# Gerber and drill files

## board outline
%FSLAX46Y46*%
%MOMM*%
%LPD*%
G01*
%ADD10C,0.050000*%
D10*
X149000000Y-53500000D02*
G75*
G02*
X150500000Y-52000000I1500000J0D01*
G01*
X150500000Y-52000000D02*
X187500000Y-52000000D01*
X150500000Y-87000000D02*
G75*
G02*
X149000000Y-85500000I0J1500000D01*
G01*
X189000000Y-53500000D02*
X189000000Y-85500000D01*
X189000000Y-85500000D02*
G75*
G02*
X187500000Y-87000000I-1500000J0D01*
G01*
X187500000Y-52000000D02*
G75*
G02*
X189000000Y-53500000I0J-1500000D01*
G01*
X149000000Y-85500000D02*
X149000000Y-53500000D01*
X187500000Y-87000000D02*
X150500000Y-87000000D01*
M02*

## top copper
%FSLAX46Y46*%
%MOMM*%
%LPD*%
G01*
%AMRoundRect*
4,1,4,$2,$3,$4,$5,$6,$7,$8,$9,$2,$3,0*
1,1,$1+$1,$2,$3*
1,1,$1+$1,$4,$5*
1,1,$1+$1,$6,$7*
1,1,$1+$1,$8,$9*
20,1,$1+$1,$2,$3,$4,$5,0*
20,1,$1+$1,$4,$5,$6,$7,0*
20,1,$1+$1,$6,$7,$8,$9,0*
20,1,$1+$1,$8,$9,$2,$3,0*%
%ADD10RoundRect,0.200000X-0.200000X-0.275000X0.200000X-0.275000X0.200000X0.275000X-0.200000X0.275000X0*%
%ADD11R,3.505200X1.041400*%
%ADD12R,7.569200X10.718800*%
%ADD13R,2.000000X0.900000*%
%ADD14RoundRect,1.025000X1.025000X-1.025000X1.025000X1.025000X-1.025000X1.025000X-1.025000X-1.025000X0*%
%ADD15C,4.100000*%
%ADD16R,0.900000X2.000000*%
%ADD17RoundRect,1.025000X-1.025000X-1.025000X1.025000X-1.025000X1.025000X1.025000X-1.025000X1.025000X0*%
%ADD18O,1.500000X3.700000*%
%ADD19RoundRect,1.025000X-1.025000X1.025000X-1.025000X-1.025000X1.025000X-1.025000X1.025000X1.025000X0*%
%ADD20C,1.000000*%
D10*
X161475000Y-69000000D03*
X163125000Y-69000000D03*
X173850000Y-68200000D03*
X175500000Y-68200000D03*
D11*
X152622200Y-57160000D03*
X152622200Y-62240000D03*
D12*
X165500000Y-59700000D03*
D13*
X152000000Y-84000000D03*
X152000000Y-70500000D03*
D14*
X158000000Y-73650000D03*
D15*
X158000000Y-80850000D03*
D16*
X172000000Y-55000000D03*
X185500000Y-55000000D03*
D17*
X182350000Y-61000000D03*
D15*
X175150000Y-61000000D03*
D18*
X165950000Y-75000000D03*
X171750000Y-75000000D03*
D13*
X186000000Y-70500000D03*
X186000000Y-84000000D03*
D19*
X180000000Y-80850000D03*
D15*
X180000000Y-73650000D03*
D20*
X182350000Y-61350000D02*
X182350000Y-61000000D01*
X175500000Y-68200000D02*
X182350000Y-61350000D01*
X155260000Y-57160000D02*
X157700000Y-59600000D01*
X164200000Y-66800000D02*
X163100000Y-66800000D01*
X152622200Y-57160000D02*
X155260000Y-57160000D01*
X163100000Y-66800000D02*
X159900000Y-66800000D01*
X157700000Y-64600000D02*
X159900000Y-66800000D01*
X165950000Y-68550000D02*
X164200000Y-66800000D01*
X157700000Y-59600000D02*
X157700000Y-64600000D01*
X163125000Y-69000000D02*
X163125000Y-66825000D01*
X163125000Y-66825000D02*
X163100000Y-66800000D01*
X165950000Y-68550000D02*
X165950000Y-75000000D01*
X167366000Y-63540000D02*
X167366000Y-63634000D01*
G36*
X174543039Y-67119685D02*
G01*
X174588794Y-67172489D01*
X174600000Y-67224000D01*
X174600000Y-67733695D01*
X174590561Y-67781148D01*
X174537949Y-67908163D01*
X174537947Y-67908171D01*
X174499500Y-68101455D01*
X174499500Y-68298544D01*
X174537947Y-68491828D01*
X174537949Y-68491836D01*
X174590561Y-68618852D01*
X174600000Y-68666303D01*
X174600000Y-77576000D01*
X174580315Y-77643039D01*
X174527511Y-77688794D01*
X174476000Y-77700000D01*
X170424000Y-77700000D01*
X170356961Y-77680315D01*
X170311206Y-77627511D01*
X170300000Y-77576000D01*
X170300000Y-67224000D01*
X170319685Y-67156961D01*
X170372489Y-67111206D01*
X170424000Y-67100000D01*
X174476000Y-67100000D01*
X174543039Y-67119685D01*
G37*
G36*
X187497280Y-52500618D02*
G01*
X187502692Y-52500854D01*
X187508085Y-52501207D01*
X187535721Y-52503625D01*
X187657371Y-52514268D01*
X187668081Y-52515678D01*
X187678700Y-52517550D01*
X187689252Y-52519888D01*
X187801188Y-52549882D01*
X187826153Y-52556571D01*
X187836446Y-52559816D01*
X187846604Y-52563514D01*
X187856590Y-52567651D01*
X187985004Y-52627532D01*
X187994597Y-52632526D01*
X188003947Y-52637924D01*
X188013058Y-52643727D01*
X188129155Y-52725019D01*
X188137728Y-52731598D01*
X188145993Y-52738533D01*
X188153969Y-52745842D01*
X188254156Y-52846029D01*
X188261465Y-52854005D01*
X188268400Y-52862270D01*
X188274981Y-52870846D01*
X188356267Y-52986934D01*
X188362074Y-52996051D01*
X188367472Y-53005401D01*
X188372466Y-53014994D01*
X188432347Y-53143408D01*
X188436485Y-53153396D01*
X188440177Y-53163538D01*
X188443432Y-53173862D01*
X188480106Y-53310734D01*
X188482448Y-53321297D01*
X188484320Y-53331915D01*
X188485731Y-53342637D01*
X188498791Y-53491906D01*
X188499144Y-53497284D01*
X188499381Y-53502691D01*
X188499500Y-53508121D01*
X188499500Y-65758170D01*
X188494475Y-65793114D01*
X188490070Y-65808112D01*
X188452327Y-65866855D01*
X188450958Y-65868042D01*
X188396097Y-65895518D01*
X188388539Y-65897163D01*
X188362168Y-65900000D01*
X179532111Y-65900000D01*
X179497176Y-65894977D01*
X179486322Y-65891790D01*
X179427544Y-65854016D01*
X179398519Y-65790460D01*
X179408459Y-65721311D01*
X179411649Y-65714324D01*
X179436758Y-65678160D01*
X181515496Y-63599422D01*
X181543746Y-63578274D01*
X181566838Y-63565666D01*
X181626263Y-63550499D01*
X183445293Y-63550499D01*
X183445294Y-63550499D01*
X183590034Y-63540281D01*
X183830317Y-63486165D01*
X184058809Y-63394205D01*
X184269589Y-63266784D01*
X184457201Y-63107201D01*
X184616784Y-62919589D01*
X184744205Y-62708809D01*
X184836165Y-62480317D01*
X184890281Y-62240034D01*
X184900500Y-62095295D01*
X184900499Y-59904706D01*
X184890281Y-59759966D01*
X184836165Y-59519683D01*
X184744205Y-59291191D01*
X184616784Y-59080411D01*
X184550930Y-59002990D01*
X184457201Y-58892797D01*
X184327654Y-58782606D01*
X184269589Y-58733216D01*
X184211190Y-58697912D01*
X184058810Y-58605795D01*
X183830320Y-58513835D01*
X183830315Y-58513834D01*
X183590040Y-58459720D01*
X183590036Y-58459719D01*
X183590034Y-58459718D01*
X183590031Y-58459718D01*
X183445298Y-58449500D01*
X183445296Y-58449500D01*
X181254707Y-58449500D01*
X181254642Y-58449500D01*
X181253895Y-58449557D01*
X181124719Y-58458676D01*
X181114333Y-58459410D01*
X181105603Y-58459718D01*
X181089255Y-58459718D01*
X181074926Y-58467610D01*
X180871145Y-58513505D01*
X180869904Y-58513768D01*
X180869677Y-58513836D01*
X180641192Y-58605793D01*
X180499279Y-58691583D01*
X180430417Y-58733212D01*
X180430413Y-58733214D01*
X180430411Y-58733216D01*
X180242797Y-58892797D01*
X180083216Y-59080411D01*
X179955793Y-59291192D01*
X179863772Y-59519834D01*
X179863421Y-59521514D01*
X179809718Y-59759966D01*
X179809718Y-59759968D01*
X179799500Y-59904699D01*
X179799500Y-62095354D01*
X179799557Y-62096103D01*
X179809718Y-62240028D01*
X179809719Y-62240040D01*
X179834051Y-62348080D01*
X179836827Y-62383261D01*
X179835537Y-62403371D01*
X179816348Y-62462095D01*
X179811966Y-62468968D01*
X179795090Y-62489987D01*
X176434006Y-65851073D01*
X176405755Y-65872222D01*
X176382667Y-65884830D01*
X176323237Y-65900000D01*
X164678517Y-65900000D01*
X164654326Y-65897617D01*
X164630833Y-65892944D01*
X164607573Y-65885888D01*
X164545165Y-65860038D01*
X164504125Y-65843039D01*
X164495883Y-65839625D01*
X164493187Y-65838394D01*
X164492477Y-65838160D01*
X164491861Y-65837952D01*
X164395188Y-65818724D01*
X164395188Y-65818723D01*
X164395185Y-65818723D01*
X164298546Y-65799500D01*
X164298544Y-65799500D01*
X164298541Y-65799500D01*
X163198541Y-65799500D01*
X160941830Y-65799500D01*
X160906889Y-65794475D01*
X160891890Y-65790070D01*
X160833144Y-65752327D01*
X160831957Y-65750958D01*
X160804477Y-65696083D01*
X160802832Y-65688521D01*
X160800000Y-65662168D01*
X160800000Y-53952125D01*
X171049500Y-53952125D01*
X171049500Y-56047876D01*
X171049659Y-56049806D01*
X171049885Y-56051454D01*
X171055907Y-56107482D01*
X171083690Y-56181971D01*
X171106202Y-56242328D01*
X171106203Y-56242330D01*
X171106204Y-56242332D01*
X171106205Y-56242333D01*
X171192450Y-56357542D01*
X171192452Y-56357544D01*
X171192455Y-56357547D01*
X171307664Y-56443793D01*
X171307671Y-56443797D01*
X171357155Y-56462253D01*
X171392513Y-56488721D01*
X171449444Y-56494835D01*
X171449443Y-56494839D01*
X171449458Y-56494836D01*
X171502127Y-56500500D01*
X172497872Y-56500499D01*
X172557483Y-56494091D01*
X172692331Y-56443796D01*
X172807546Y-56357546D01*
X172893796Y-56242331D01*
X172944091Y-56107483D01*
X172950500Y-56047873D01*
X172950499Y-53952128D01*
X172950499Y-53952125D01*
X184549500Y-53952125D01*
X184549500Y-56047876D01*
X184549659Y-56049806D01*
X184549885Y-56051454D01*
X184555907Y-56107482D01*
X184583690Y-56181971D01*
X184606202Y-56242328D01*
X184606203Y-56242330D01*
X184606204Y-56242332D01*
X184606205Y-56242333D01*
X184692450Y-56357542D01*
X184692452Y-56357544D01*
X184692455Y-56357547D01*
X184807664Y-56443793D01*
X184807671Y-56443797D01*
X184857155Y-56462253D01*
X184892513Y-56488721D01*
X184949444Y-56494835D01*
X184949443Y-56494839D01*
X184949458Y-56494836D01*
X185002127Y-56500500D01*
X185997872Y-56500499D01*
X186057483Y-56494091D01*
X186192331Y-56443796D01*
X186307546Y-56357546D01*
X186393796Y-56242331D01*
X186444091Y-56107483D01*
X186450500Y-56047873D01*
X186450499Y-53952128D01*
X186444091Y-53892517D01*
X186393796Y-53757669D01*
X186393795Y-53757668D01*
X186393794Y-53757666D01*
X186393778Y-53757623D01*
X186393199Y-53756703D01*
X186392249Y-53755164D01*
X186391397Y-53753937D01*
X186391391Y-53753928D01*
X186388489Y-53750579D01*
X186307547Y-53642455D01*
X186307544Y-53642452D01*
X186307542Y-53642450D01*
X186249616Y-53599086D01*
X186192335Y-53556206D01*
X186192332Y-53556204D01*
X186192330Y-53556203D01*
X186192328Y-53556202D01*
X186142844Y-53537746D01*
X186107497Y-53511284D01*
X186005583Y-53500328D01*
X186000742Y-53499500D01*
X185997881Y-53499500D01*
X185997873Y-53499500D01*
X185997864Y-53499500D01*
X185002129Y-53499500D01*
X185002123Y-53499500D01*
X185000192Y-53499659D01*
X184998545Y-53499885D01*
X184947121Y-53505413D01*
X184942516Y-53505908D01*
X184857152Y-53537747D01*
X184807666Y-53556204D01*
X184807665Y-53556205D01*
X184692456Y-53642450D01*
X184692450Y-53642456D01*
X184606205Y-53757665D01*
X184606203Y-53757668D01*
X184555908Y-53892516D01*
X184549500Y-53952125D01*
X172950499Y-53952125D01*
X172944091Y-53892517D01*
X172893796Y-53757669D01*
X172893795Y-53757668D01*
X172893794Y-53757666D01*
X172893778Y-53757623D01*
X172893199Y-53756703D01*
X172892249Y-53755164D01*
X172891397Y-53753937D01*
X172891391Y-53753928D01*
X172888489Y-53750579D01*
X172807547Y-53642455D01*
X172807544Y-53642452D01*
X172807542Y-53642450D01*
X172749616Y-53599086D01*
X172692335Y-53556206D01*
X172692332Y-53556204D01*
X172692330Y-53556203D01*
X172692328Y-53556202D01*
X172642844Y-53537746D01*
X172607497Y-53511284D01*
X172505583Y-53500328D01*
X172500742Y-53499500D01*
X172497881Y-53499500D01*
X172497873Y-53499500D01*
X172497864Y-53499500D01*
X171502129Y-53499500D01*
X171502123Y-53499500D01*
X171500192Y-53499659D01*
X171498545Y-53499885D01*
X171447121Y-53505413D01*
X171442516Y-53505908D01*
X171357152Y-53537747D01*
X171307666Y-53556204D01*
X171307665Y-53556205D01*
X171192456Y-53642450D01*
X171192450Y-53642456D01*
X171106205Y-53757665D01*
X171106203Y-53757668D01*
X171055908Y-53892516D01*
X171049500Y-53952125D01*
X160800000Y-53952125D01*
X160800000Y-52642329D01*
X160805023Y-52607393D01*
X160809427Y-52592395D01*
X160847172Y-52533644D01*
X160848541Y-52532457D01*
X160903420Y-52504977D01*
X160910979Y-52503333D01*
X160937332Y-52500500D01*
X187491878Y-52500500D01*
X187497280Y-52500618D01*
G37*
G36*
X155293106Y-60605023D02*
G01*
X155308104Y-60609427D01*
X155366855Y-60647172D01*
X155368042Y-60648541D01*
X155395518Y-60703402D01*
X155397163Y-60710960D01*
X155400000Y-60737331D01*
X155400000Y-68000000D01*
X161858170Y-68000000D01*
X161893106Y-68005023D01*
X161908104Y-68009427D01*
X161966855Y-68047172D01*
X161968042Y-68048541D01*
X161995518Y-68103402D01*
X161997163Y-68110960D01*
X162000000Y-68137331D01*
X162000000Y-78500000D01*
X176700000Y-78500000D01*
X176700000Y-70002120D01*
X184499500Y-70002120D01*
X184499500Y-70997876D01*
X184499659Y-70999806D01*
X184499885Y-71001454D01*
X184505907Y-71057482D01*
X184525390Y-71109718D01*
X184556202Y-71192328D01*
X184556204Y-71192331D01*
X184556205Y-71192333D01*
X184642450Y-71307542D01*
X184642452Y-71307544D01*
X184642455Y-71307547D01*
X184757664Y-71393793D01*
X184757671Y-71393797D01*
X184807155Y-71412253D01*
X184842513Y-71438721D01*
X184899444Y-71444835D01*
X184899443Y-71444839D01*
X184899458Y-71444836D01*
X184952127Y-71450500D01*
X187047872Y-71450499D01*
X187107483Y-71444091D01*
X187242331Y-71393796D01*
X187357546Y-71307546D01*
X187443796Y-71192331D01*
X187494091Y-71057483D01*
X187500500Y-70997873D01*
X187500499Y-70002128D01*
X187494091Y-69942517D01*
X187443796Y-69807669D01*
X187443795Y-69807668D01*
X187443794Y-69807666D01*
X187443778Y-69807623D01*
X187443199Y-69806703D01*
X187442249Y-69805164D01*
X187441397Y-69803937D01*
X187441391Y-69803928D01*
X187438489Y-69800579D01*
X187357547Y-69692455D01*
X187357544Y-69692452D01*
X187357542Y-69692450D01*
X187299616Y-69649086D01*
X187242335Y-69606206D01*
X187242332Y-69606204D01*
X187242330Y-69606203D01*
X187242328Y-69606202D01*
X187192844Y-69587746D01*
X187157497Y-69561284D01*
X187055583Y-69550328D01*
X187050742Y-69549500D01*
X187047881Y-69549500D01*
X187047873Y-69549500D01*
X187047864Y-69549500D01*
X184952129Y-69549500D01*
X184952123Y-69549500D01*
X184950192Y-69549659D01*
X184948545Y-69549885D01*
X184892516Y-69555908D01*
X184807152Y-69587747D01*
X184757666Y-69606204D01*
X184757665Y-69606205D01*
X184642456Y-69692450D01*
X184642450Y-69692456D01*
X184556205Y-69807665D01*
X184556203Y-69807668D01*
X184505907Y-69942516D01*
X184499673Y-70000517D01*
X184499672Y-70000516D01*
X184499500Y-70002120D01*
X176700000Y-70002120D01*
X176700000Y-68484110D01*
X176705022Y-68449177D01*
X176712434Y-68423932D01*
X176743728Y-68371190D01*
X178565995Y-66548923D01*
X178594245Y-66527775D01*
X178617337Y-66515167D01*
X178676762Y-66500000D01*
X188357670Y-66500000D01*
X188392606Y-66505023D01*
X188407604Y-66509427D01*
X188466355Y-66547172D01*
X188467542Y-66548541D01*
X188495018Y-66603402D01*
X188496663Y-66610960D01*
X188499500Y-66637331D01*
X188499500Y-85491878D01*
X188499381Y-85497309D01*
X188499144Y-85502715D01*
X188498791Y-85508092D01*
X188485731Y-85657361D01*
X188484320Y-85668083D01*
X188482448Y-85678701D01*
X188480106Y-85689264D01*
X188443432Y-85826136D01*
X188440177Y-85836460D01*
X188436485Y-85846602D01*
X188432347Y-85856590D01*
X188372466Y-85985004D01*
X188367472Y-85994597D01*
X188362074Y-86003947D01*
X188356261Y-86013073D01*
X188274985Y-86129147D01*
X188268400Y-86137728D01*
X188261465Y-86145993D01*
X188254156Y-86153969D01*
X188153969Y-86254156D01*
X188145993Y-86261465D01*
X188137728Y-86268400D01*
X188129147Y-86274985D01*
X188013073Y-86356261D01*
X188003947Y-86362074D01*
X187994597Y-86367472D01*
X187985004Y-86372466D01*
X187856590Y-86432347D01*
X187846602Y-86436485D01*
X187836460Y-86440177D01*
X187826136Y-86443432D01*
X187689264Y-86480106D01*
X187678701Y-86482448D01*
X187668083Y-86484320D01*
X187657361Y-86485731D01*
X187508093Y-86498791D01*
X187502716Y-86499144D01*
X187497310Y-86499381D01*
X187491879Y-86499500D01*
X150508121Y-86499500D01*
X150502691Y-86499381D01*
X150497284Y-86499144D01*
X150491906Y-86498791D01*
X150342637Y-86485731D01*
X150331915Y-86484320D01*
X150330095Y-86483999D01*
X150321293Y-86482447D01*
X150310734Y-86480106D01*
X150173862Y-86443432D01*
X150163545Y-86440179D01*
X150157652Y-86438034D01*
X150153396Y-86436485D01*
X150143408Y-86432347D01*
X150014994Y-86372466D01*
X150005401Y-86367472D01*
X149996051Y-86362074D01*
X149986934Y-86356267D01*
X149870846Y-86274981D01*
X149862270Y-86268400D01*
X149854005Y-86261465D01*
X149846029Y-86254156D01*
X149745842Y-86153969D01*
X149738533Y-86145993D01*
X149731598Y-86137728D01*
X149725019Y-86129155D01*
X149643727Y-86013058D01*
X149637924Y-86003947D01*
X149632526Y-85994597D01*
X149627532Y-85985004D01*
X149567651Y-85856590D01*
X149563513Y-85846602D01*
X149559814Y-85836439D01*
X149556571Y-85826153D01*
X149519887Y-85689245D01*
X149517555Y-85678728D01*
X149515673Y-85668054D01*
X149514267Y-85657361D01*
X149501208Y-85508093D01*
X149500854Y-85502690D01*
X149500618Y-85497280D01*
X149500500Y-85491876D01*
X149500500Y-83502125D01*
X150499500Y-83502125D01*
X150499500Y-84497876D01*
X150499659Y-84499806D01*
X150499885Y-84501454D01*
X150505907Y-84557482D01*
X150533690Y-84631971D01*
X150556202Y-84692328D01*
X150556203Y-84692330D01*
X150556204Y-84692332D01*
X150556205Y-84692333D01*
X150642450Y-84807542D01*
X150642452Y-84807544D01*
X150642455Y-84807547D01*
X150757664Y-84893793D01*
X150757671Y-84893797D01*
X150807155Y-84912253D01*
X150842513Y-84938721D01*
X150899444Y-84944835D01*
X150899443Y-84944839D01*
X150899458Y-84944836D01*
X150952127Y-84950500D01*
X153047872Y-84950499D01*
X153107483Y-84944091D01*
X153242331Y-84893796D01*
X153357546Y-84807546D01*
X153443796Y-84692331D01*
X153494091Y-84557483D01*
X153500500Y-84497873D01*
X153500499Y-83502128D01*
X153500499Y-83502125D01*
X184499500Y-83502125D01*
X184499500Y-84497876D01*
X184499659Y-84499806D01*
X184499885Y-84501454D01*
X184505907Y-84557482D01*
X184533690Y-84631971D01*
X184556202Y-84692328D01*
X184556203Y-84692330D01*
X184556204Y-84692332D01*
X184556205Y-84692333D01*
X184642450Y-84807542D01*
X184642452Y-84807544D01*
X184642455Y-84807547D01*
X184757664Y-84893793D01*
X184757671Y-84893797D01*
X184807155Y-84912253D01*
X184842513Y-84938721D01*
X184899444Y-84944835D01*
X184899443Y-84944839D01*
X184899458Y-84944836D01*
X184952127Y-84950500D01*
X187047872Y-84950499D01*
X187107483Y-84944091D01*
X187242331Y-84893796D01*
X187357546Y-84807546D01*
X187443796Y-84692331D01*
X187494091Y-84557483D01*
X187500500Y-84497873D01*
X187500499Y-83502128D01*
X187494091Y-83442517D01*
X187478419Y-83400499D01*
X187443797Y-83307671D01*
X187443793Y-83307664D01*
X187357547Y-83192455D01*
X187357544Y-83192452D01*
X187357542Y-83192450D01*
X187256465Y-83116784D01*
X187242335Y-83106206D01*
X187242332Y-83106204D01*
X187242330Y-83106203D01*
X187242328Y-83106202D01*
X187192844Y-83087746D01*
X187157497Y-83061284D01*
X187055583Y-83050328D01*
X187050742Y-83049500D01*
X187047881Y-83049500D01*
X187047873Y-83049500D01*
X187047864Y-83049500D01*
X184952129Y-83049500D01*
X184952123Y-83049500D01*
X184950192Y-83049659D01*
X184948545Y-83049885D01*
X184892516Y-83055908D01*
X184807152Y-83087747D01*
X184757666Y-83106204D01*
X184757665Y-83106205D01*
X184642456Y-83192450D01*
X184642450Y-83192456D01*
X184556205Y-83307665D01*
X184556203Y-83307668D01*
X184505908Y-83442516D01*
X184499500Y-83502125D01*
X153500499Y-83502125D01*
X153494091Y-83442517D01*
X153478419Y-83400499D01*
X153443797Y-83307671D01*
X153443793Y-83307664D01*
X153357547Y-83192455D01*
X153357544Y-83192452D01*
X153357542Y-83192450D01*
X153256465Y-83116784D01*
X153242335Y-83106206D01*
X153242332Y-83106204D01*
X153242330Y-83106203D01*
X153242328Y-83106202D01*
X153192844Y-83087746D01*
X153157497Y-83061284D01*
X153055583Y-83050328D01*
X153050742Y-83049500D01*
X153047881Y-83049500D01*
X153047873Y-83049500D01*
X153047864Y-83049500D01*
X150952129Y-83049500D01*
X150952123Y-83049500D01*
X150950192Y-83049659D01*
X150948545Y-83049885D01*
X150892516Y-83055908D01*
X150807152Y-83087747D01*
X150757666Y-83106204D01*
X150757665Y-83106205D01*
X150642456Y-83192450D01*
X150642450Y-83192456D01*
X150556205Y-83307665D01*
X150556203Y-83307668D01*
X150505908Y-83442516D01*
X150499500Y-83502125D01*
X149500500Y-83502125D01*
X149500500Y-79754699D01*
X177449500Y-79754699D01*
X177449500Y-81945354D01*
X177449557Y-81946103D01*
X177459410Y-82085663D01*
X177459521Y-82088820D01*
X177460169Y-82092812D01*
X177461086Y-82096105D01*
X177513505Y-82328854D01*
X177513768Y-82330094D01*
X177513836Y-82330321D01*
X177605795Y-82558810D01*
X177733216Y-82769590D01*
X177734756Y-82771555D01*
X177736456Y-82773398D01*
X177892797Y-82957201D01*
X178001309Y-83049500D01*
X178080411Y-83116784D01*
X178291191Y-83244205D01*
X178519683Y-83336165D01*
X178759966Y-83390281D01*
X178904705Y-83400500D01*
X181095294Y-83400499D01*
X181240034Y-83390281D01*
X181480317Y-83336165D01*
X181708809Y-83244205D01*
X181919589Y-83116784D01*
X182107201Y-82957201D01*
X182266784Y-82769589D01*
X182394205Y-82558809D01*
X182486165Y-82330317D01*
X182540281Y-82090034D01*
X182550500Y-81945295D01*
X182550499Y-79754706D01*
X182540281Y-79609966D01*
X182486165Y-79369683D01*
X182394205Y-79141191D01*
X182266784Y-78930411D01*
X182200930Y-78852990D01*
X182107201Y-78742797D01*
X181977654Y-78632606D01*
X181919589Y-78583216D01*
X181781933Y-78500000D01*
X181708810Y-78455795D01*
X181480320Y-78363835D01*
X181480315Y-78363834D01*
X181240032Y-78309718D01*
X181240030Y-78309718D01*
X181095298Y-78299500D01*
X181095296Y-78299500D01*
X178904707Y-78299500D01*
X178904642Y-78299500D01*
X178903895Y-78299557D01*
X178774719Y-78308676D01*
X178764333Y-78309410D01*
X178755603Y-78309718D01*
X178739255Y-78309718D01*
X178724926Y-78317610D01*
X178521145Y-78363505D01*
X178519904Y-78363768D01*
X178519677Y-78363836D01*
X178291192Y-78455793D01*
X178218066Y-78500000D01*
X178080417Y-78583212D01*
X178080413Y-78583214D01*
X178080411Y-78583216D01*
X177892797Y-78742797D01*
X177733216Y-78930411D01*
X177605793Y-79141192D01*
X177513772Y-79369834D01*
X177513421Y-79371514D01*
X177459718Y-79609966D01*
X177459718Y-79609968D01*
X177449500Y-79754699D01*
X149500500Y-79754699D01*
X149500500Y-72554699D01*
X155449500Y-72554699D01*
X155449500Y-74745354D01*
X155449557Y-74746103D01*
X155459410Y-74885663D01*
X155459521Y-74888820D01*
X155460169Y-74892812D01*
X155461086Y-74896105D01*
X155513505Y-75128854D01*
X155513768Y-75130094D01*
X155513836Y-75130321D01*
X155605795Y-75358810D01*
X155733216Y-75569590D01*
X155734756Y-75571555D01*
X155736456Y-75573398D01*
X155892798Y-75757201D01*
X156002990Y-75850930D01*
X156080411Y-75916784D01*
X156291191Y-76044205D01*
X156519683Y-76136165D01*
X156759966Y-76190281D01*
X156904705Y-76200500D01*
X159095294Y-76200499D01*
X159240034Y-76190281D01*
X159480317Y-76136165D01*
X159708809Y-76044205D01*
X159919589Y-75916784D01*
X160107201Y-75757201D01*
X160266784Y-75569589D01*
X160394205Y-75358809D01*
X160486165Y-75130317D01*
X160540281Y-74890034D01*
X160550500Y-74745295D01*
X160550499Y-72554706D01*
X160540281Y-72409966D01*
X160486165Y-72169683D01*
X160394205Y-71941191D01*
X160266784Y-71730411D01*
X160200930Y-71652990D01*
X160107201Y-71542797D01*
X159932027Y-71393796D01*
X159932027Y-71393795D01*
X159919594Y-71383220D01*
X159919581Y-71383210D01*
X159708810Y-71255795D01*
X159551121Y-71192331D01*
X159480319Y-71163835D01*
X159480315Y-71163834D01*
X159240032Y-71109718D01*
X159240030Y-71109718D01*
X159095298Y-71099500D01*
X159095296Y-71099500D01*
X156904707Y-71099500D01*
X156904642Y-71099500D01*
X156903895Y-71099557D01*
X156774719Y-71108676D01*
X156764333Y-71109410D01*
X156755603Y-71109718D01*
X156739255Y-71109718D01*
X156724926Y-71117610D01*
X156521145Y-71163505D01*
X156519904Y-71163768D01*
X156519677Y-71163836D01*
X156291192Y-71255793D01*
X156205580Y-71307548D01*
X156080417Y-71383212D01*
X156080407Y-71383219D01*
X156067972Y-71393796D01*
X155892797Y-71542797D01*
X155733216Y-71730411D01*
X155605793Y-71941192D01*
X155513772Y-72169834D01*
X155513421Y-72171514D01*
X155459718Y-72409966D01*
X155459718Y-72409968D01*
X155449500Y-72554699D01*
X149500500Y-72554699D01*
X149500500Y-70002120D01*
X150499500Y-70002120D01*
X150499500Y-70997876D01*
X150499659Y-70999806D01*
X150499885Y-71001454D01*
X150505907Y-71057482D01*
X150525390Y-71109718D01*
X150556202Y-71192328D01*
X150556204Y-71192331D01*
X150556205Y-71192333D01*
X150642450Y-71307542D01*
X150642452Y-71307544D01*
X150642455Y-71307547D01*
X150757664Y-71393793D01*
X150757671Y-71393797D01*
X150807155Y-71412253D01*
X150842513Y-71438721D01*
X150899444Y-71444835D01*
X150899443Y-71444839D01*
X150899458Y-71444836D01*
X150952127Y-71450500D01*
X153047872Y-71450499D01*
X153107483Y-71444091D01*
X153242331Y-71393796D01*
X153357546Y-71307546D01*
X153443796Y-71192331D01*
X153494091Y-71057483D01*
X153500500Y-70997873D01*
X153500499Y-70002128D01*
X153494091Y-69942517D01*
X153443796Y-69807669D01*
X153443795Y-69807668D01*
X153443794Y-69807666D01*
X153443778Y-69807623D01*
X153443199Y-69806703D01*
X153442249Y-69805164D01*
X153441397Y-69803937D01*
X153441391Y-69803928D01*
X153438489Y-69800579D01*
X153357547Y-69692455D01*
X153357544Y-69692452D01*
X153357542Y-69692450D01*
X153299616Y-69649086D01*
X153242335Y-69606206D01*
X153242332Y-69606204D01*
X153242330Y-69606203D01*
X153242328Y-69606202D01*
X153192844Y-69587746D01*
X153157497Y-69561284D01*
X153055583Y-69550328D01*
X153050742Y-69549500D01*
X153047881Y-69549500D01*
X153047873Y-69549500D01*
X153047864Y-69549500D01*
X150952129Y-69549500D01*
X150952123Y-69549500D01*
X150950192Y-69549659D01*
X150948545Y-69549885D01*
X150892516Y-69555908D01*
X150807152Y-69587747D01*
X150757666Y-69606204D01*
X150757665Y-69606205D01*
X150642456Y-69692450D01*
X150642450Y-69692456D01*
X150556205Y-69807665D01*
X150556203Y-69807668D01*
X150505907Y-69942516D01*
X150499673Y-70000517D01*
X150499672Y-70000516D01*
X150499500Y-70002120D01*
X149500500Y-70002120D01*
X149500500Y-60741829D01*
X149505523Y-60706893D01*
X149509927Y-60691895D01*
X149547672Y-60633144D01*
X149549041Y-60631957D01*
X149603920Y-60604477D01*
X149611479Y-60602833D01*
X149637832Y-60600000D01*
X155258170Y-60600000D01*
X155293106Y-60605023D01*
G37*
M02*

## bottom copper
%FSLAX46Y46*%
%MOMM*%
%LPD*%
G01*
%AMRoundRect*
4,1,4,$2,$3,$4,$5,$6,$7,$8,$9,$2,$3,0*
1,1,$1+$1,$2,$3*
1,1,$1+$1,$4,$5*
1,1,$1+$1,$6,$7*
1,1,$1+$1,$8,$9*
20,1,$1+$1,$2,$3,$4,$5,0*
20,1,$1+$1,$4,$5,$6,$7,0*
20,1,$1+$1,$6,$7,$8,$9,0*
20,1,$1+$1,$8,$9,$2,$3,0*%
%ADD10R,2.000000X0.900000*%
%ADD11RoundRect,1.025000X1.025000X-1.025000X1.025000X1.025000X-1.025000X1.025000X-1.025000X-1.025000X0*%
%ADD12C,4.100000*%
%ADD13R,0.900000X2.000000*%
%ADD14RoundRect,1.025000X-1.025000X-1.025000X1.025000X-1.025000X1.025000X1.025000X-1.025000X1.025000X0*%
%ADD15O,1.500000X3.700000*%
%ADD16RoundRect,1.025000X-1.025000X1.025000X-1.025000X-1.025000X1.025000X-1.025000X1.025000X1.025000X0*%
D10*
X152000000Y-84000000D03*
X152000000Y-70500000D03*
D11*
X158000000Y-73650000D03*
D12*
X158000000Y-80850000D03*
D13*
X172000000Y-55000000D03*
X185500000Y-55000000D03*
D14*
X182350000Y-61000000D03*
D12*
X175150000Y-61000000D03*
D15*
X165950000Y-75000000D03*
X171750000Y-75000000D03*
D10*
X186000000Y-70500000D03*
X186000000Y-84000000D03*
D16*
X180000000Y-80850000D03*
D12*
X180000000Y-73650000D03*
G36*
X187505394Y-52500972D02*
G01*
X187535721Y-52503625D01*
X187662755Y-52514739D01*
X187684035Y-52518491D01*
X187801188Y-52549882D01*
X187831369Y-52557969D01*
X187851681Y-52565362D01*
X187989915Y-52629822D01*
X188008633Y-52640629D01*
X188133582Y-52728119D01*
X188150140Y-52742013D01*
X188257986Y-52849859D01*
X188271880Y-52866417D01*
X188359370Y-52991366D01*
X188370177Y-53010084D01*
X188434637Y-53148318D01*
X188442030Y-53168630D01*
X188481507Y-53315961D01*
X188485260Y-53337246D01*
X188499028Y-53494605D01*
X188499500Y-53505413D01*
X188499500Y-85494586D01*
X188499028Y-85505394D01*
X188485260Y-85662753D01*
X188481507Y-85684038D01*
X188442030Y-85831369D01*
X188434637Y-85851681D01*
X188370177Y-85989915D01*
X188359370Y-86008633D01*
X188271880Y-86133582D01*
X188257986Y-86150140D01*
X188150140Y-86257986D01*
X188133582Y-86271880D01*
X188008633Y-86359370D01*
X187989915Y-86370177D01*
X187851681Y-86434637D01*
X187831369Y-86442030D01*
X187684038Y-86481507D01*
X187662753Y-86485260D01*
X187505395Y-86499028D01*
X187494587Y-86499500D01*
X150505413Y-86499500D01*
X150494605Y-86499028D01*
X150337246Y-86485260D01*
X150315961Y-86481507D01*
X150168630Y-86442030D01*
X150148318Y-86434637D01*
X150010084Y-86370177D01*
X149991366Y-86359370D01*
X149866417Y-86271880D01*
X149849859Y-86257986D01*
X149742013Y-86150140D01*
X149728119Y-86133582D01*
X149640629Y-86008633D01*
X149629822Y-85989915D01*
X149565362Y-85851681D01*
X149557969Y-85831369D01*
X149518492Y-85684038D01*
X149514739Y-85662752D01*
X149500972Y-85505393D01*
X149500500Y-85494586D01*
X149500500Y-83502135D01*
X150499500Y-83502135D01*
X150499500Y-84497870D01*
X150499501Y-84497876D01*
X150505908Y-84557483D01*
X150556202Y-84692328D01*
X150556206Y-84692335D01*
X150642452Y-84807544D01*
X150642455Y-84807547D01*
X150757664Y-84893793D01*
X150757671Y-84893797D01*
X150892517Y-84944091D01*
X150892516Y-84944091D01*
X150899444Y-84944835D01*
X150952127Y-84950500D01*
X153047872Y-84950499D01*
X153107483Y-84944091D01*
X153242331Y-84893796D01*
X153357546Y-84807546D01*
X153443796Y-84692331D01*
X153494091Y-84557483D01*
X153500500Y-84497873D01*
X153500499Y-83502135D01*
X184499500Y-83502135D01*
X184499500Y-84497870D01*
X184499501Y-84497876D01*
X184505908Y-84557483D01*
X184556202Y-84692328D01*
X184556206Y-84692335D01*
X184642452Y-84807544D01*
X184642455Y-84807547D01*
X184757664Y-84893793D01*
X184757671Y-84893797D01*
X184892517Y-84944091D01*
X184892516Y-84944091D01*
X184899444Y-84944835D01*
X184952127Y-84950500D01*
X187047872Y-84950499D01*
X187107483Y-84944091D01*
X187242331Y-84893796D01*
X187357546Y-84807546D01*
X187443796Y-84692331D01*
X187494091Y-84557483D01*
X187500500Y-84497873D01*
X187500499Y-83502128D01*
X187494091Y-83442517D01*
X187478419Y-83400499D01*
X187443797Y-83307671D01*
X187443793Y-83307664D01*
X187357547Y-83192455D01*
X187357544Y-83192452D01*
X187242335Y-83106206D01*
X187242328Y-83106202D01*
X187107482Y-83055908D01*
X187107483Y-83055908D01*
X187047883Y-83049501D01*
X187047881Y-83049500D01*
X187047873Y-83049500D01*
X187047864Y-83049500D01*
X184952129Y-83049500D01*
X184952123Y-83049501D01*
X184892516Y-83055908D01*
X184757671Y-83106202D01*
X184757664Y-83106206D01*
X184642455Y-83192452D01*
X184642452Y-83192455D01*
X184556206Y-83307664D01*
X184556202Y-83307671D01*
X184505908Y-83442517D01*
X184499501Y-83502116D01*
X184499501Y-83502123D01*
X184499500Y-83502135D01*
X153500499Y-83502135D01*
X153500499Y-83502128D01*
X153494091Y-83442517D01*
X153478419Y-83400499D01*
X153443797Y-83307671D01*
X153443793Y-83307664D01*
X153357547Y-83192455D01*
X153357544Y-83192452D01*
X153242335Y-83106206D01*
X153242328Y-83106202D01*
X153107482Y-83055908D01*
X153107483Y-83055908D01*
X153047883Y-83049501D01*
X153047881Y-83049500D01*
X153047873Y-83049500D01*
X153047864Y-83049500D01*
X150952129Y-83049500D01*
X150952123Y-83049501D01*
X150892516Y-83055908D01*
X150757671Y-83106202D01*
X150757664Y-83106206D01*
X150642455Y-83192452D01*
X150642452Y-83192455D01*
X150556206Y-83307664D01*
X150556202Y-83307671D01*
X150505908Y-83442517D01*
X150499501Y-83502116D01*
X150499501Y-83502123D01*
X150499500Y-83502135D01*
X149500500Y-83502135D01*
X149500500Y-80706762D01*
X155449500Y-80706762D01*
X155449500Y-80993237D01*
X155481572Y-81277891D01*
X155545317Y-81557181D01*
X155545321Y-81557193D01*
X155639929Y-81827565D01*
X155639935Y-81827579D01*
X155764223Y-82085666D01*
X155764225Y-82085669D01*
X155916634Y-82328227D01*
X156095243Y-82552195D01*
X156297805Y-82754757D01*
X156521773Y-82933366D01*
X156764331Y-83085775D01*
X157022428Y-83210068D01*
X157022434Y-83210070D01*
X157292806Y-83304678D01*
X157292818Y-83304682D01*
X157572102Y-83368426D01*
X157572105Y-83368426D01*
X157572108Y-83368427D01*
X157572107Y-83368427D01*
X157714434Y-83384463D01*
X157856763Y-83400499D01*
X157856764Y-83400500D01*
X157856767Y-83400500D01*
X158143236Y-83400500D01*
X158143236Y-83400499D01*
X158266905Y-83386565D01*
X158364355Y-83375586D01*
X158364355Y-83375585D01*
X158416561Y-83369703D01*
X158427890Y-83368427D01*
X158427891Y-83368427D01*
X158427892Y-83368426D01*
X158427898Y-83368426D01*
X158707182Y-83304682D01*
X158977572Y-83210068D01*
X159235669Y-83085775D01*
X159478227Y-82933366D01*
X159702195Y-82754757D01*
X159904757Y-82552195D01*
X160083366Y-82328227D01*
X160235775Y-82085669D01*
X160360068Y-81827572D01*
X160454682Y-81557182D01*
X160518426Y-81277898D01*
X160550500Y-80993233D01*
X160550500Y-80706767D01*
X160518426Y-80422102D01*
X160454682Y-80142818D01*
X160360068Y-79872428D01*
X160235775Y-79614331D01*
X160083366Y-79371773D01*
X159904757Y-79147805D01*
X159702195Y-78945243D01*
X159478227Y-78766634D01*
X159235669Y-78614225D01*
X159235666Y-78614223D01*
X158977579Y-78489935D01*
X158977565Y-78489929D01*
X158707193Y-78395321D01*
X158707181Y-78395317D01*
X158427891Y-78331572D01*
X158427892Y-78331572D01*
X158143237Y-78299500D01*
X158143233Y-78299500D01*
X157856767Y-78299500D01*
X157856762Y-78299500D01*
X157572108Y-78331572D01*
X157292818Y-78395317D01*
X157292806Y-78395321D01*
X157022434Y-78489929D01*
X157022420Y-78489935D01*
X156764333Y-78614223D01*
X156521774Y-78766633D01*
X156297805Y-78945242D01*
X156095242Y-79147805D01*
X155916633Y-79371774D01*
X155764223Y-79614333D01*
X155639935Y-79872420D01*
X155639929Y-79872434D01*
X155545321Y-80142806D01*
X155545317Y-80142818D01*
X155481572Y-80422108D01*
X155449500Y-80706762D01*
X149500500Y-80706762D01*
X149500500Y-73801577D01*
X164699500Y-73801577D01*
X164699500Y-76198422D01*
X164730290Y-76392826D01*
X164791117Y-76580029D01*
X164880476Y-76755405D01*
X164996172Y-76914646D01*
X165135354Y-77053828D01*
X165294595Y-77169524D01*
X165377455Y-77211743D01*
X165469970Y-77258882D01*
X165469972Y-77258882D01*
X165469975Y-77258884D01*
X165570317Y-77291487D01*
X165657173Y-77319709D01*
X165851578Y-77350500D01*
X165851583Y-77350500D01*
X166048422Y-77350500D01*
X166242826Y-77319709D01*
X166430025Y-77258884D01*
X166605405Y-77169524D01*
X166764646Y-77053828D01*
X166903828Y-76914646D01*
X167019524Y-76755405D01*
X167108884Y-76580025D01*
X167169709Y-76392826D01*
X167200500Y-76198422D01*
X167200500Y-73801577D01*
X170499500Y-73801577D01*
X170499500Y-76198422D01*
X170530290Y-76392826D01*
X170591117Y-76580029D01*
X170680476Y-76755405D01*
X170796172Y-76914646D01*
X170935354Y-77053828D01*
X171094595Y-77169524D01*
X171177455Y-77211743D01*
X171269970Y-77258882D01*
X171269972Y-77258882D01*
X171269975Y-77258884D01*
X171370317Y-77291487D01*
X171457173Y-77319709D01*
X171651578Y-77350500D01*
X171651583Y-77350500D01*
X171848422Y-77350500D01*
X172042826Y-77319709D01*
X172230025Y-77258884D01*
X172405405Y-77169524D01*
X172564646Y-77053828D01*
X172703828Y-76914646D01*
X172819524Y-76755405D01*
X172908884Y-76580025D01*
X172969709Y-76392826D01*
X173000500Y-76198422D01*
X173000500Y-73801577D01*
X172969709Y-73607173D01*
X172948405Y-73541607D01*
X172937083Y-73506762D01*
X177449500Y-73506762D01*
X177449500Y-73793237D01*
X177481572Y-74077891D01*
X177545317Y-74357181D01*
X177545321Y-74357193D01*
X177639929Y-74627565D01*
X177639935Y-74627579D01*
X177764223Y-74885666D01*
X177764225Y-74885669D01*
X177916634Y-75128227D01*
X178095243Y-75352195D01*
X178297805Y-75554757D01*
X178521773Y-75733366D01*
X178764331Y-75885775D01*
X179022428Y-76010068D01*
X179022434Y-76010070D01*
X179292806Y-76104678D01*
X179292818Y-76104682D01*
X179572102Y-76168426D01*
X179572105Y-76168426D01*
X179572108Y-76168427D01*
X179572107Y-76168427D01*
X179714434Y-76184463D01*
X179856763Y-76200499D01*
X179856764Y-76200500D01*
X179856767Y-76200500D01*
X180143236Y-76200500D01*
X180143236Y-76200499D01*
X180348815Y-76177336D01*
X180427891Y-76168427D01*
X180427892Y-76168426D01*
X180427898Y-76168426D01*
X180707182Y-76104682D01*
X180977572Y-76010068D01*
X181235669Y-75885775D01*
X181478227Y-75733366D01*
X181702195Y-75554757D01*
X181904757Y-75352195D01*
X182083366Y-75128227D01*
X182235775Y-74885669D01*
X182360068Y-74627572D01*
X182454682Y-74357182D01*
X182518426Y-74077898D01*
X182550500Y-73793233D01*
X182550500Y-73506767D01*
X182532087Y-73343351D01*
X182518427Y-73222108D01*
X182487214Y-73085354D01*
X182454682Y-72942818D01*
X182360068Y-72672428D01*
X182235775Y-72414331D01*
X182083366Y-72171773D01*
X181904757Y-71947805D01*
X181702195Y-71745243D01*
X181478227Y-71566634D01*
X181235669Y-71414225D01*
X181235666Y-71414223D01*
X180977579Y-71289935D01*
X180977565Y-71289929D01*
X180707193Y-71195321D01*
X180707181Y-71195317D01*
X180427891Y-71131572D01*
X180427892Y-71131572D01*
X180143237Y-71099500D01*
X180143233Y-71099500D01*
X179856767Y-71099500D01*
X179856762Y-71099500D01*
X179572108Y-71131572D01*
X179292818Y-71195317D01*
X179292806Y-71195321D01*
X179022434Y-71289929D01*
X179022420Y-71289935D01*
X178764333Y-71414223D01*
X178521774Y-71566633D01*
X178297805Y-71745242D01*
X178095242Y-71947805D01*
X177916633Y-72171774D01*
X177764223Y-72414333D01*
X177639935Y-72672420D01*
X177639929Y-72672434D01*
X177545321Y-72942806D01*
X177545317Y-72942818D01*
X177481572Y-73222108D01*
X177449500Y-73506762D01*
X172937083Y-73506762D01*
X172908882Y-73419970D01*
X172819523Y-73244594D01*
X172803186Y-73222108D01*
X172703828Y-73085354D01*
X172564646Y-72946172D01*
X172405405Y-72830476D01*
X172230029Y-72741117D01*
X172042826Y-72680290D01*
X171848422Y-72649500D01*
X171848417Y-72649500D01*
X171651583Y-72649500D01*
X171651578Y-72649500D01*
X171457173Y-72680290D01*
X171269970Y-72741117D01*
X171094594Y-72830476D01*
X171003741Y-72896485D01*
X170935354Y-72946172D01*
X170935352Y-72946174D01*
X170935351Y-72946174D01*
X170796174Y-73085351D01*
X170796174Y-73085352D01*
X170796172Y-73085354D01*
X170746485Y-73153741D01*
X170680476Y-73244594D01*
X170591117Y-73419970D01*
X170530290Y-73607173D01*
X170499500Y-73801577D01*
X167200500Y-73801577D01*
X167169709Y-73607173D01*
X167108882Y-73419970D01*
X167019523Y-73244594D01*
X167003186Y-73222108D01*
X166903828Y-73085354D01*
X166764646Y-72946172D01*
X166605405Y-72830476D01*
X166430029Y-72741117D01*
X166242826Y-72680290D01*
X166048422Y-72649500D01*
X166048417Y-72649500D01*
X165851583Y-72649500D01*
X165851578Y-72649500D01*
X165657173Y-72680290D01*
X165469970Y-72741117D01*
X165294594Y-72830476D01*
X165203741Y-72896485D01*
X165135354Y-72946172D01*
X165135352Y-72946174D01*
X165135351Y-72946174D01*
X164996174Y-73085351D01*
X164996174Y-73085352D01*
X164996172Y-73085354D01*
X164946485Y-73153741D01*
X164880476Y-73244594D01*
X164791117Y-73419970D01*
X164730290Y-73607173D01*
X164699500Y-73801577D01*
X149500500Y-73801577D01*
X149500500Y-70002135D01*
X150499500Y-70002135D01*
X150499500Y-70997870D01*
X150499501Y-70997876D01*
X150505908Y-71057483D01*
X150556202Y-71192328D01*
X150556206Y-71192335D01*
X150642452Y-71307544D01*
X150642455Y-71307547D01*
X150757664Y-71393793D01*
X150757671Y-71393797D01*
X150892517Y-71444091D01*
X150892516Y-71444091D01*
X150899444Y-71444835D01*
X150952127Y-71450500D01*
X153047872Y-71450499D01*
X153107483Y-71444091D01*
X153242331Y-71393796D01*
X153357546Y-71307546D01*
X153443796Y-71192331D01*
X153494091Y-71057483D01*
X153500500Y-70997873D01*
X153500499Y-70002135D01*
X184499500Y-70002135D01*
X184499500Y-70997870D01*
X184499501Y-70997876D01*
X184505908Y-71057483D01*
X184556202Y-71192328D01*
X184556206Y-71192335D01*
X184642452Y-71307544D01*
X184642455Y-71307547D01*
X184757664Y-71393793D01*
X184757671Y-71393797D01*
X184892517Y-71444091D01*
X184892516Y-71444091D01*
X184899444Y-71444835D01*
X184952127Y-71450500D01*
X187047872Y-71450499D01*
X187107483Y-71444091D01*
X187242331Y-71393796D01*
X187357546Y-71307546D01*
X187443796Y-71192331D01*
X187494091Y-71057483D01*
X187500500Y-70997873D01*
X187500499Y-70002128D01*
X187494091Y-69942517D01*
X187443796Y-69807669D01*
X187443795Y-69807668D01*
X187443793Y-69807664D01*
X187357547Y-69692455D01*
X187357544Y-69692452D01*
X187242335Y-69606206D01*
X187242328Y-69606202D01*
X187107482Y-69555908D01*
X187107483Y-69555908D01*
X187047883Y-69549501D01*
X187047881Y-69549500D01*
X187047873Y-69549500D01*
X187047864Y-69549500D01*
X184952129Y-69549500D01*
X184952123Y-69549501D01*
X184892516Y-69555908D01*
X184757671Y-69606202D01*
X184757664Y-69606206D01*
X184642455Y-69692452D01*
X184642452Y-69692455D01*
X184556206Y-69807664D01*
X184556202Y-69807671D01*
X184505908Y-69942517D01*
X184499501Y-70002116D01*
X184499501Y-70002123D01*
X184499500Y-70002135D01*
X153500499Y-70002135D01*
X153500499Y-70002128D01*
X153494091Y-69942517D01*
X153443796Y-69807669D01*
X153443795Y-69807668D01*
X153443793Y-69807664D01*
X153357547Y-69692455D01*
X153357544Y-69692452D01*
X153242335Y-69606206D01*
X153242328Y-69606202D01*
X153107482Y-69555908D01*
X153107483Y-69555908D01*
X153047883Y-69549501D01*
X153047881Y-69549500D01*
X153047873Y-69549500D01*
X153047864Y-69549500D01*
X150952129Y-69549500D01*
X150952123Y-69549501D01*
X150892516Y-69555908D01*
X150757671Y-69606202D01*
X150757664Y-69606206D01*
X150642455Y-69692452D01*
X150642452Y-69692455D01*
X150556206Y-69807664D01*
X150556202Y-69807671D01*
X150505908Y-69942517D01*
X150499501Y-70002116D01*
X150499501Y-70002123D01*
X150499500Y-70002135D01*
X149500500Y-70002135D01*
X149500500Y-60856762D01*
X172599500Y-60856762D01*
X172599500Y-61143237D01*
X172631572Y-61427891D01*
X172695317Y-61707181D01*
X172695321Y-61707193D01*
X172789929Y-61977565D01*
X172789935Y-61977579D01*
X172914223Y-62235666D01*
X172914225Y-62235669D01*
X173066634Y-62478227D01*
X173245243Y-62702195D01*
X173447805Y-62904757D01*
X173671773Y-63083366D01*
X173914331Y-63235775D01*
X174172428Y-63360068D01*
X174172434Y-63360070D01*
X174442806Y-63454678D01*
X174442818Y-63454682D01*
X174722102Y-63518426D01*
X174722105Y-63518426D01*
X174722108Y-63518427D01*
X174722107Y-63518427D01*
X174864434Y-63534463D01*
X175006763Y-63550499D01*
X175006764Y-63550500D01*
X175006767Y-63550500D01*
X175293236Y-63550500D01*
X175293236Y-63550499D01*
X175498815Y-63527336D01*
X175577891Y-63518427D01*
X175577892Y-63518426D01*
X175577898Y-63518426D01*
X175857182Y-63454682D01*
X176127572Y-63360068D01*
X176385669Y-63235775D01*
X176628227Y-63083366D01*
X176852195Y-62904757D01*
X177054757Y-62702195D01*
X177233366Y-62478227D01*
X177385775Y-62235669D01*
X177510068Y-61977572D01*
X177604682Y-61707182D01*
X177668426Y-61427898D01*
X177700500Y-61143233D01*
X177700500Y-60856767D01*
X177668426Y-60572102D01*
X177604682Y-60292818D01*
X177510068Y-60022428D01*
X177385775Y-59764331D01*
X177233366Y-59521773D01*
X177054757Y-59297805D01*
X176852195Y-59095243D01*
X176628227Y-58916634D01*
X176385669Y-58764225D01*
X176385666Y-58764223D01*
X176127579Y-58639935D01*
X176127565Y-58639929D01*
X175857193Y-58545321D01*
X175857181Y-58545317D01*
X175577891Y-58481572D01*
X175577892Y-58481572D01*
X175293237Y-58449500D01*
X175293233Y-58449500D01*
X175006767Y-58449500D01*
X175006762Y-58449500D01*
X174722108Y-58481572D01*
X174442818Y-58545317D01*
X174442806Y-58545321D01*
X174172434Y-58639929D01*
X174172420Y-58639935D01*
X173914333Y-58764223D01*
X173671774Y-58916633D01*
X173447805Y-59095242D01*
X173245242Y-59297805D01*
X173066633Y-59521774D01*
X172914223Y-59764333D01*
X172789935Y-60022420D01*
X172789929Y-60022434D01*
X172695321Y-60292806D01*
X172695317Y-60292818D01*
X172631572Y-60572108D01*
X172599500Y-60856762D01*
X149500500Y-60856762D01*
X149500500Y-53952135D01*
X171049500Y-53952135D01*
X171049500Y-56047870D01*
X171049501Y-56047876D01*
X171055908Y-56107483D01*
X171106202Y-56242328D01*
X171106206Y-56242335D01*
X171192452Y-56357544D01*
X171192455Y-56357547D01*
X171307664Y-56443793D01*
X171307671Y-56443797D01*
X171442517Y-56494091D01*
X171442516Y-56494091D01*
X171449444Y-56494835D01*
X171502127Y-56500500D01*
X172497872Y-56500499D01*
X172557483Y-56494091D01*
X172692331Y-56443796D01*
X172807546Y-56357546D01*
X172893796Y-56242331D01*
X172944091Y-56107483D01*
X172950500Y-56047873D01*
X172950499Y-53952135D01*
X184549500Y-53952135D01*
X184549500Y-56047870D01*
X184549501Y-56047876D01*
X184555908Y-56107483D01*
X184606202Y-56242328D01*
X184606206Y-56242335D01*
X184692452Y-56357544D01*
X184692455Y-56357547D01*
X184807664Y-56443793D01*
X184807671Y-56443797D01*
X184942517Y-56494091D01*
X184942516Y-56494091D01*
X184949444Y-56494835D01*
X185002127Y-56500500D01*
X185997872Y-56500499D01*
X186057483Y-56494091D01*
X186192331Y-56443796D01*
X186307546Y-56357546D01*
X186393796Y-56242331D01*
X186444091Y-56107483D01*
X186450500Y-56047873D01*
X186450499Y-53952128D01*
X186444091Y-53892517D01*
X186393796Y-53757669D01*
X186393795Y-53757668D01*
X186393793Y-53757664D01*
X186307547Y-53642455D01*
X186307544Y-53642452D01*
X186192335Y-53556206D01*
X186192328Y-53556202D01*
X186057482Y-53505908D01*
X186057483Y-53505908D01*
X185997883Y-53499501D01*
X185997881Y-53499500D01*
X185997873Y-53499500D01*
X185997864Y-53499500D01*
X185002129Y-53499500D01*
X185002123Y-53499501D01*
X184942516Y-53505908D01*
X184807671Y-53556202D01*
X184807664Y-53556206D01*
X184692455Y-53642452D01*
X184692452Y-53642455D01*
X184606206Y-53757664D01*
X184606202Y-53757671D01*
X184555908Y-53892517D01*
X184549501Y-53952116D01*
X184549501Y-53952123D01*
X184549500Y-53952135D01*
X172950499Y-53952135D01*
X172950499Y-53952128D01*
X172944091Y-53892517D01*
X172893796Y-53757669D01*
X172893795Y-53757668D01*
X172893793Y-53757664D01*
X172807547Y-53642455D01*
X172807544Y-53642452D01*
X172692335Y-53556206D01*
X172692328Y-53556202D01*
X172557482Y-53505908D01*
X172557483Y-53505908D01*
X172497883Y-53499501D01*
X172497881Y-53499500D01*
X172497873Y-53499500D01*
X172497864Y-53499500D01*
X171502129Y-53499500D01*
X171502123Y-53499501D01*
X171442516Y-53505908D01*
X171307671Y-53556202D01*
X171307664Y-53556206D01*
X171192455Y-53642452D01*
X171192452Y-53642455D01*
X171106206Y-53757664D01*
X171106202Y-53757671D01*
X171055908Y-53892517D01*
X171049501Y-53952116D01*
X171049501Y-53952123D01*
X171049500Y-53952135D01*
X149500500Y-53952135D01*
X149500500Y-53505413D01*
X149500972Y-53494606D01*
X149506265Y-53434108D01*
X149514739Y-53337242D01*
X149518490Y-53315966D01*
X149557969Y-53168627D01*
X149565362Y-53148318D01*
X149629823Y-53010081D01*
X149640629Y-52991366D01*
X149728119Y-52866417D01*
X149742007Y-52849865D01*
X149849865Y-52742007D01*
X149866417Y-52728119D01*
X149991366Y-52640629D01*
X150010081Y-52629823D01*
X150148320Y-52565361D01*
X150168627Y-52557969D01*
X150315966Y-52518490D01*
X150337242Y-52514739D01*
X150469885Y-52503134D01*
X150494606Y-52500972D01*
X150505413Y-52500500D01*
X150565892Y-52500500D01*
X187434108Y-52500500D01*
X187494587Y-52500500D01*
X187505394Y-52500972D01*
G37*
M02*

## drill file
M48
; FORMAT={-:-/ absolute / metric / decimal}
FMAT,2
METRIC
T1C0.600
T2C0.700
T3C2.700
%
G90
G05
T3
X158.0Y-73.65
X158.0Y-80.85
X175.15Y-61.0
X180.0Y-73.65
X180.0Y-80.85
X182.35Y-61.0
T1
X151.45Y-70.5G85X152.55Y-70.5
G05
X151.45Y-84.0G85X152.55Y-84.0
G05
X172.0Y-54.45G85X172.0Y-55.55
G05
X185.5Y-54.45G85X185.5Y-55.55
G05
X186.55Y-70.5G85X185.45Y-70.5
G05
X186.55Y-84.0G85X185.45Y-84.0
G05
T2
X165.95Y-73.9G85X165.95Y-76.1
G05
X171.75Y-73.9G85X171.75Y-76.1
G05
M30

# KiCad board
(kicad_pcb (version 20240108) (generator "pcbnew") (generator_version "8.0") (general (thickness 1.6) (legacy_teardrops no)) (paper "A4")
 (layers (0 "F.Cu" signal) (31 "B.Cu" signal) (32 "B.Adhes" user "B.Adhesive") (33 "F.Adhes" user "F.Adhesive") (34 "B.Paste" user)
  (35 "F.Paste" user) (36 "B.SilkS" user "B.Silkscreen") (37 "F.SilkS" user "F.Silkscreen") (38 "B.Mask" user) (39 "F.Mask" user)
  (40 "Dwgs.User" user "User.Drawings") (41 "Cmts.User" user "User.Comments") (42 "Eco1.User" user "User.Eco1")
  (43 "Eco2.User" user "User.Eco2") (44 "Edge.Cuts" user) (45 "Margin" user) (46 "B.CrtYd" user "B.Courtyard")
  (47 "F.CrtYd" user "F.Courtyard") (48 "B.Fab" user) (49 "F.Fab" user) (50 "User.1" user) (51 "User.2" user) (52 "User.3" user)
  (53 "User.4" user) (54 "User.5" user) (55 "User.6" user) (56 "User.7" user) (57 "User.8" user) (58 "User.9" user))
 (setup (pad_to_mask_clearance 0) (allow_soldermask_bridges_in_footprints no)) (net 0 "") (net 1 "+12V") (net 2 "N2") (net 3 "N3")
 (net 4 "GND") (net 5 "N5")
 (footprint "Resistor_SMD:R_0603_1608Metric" (layer "F.Cu") (at 162.3 69)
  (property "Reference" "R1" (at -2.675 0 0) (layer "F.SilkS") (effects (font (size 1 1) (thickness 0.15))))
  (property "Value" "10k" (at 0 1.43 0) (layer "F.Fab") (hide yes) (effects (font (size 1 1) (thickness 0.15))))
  (pad "1" smd roundrect (at -0.825 0) (size 0.8 0.95) (layers "F.Cu" "F.Paste" "F.Mask") (roundrect_rratio 0.25) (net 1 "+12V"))
  (pad "2" smd roundrect (at 0.825 0) (size 0.8 0.95) (layers "F.Cu" "F.Paste" "F.Mask") (roundrect_rratio 0.25) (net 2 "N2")))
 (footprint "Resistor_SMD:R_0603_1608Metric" (layer "F.Cu") (at 174.675 68.2)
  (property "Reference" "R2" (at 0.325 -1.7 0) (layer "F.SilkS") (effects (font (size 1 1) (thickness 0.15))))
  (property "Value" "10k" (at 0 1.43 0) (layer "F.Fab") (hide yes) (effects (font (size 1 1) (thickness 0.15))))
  (pad "1" smd roundrect (at -0.825 0) (size 0.8 0.95) (layers "F.Cu" "F.Paste" "F.Mask") (roundrect_rratio 0.25) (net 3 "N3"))
  (pad "2" smd roundrect (at 0.825 0) (size 0.8 0.95) (layers "F.Cu" "F.Paste" "F.Mask") (roundrect_rratio 0.25) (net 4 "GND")))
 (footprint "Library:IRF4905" (layer "F.Cu") (at 162.2742 59.7 -90)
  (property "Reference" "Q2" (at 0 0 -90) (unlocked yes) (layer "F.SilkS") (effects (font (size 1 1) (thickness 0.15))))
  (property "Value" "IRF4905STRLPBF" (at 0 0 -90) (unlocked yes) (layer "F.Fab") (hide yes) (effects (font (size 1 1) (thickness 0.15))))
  (pad "1" smd rect (at -2.54 9.652 270) (size 1.0414 3.5052) (layers "F.Cu" "F.Paste" "F.Mask") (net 2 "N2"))
  (pad "2" smd rect (at 2.54 9.652 270) (size 1.0414 3.5052) (layers "F.Cu" "F.Paste" "F.Mask") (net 1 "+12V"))
  (pad "3" smd rect (at 0 -3.2258 270) (size 10.7188 7.5692) (layers "F.Cu" "F.Paste" "F.Mask") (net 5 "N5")))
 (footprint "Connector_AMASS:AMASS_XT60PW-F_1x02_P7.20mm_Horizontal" (layer "F.Cu") (at 158 73.65 90)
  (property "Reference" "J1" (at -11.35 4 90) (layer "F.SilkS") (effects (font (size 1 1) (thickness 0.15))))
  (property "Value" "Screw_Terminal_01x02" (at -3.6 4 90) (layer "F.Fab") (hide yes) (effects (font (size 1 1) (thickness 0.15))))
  (pad "" thru_hole rect (at -10.35 -6 90) (size 0.9 2) (drill oval 0.6 1.7) (layers "*.Cu" "*.Mask") (remove_unused_layers no))
  (pad "" thru_hole rect (at 3.15 -6 90) (size 0.9 2) (drill oval 0.6 1.7) (layers "*.Cu" "*.Mask") (remove_unused_layers no))
  (pad "1" thru_hole roundrect (at 0 0 90) (size 4.1 4.1) (drill 2.7) (layers "*.Cu" "*.Mask") (remove_unused_layers no)
   (roundrect_rratio 0.25) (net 4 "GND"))
  (pad "2" thru_hole circle (at -7.2 0 90) (size 4.1 4.1) (drill 2.7) (layers "*.Cu" "*.Mask") (remove_unused_layers no) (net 1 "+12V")))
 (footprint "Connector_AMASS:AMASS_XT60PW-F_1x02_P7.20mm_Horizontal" (layer "F.Cu") (at 182.35 61)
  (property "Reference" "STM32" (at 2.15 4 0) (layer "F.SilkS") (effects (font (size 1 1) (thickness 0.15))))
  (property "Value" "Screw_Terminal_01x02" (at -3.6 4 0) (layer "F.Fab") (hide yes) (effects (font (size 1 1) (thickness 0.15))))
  (pad "" thru_hole rect (at -10.35 -6) (size 0.9 2) (drill oval 0.6 1.7) (layers "*.Cu" "*.Mask") (remove_unused_layers no))
  (pad "" thru_hole rect (at 3.15 -6) (size 0.9 2) (drill oval 0.6 1.7) (layers "*.Cu" "*.Mask") (remove_unused_layers no))
  (pad "1" thru_hole roundrect (at 0 0) (size 4.1 4.1) (drill 2.7) (layers "*.Cu" "*.Mask") (remove_unused_layers no)
   (roundrect_rratio 0.25) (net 4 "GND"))
  (pad "2" thru_hole circle (at -7.2 0) (size 4.1 4.1) (drill 2.7) (layers "*.Cu" "*.Mask") (remove_unused_layers no) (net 5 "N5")))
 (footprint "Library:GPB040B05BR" (layer "F.Cu") (at 166.54 79.66)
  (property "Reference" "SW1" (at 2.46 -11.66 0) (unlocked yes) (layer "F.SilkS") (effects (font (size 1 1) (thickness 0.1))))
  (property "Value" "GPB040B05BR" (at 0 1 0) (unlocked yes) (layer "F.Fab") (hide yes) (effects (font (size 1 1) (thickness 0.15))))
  (pad "1" thru_hole oval (at -0.59 -4.66) (size 1.5 3.7) (drill oval 0.7 2.9) (layers "*.Cu" "*.Mask") (remove_unused_layers no)
   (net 2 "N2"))
  (pad "2" thru_hole oval (at 5.21 -4.66) (size 1.5 3.7) (drill oval 0.7 2.9) (layers "*.Cu" "*.Mask") (remove_unused_layers no)
   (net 3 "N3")))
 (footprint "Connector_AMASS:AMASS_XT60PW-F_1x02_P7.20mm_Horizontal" (layer "F.Cu") (at 180 80.85 -90)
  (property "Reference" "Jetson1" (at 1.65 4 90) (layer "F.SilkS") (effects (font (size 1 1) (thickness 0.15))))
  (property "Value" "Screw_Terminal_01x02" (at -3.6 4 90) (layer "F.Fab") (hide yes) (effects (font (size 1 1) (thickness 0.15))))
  (pad "" thru_hole rect (at -10.35 -6 270) (size 0.9 2) (drill oval 0.6 1.7) (layers "*.Cu" "*.Mask") (remove_unused_layers no))
  (pad "" thru_hole rect (at 3.15 -6 270) (size 0.9 2) (drill oval 0.6 1.7) (layers "*.Cu" "*.Mask") (remove_unused_layers no))
  (pad "1" thru_hole roundrect (at 0 0 270) (size 4.1 4.1) (drill 2.7) (layers "*.Cu" "*.Mask") (remove_unused_layers no)
   (roundrect_rratio 0.25) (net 4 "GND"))
  (pad "2" thru_hole circle (at -7.2 0 270) (size 4.1 4.1) (drill 2.7) (layers "*.Cu" "*.Mask") (remove_unused_layers no) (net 1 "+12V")))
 (gr_arc (start 149 53.5) (mid 149.43934 52.43934) (end 150.5 52) (stroke (width 0.05) (type default)) (layer "Edge.Cuts"))
 (gr_line (start 150.5 52) (end 187.5 52) (stroke (width 0.05) (type default)) (layer "Edge.Cuts"))
 (gr_arc (start 150.5 87) (mid 149.43934 86.56066) (end 149 85.5) (stroke (width 0.05) (type default)) (layer "Edge.Cuts"))
 (gr_line (start 189 53.5) (end 189 85.5) (stroke (width 0.05) (type default)) (layer "Edge.Cuts"))
 (gr_arc (start 189 85.5) (mid 188.56066 86.56066) (end 187.5 87) (stroke (width 0.05) (type default)) (layer "Edge.Cuts"))
 (gr_arc (start 187.5 52) (mid 188.56066 52.43934) (end 189 53.5) (stroke (width 0.05) (type default)) (layer "Edge.Cuts"))
 (gr_line (start 149 85.5) (end 149 53.5) (stroke (width 0.05) (type default)) (layer "Edge.Cuts"))
 (gr_line (start 187.5 87) (end 150.5 87) (stroke (width 0.05) (type default)) (layer "Edge.Cuts"))
 (segment (start 182.35 61.35) (end 182.35 61) (width 1) (layer "F.Cu") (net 4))
 (segment (start 175.5 68.2) (end 182.35 61.35) (width 1) (layer "F.Cu") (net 4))
 (segment (start 155.26 57.16) (end 157.7 59.6) (width 1) (layer "F.Cu") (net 2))
 (segment (start 164.2 66.8) (end 163.1 66.8) (width 1) (layer "F.Cu") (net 2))
 (segment (start 152.6222 57.16) (end 155.26 57.16) (width 1) (layer "F.Cu") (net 2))
 (segment (start 163.1 66.8) (end 159.9 66.8) (width 1) (layer "F.Cu") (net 2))
 (segment (start 157.7 64.6) (end 159.9 66.8) (width 1) (layer "F.Cu") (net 2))
 (segment (start 165.95 68.55) (end 164.2 66.8) (width 1) (layer "F.Cu") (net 2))
 (segment (start 157.7 59.6) (end 157.7 64.6) (width 1) (layer "F.Cu") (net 2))
 (segment (start 163.125 69) (end 163.125 66.825) (width 1) (layer "F.Cu") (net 2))
 (segment (start 163.125 66.825) (end 163.1 66.8) (width 1) (layer "F.Cu") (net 2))
 (segment (start 165.95 68.55) (end 165.95 75) (width 1) (layer "F.Cu") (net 2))
 (segment (start 167.366 63.54) (end 167.366 63.634) (width 1) (layer "F.Cu") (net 5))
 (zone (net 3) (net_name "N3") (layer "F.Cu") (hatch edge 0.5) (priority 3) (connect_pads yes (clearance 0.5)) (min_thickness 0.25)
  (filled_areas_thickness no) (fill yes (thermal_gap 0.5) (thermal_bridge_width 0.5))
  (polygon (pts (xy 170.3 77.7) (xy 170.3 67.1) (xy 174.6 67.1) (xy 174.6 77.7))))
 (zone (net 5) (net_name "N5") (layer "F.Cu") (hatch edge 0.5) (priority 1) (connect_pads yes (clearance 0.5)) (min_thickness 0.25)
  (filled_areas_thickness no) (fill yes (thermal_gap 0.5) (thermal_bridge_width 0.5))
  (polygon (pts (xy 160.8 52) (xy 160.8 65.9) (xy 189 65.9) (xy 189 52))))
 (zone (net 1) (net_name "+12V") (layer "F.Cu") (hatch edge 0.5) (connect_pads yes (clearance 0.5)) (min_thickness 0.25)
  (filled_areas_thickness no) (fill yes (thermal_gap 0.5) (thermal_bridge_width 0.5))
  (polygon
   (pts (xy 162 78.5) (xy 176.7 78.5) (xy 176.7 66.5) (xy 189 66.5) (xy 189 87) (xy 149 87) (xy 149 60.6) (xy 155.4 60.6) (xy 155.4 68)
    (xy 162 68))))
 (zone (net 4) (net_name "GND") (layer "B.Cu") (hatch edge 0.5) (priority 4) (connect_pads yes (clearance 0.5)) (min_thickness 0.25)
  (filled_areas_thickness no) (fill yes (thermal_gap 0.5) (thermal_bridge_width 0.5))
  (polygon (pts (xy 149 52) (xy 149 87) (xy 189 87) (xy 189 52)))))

